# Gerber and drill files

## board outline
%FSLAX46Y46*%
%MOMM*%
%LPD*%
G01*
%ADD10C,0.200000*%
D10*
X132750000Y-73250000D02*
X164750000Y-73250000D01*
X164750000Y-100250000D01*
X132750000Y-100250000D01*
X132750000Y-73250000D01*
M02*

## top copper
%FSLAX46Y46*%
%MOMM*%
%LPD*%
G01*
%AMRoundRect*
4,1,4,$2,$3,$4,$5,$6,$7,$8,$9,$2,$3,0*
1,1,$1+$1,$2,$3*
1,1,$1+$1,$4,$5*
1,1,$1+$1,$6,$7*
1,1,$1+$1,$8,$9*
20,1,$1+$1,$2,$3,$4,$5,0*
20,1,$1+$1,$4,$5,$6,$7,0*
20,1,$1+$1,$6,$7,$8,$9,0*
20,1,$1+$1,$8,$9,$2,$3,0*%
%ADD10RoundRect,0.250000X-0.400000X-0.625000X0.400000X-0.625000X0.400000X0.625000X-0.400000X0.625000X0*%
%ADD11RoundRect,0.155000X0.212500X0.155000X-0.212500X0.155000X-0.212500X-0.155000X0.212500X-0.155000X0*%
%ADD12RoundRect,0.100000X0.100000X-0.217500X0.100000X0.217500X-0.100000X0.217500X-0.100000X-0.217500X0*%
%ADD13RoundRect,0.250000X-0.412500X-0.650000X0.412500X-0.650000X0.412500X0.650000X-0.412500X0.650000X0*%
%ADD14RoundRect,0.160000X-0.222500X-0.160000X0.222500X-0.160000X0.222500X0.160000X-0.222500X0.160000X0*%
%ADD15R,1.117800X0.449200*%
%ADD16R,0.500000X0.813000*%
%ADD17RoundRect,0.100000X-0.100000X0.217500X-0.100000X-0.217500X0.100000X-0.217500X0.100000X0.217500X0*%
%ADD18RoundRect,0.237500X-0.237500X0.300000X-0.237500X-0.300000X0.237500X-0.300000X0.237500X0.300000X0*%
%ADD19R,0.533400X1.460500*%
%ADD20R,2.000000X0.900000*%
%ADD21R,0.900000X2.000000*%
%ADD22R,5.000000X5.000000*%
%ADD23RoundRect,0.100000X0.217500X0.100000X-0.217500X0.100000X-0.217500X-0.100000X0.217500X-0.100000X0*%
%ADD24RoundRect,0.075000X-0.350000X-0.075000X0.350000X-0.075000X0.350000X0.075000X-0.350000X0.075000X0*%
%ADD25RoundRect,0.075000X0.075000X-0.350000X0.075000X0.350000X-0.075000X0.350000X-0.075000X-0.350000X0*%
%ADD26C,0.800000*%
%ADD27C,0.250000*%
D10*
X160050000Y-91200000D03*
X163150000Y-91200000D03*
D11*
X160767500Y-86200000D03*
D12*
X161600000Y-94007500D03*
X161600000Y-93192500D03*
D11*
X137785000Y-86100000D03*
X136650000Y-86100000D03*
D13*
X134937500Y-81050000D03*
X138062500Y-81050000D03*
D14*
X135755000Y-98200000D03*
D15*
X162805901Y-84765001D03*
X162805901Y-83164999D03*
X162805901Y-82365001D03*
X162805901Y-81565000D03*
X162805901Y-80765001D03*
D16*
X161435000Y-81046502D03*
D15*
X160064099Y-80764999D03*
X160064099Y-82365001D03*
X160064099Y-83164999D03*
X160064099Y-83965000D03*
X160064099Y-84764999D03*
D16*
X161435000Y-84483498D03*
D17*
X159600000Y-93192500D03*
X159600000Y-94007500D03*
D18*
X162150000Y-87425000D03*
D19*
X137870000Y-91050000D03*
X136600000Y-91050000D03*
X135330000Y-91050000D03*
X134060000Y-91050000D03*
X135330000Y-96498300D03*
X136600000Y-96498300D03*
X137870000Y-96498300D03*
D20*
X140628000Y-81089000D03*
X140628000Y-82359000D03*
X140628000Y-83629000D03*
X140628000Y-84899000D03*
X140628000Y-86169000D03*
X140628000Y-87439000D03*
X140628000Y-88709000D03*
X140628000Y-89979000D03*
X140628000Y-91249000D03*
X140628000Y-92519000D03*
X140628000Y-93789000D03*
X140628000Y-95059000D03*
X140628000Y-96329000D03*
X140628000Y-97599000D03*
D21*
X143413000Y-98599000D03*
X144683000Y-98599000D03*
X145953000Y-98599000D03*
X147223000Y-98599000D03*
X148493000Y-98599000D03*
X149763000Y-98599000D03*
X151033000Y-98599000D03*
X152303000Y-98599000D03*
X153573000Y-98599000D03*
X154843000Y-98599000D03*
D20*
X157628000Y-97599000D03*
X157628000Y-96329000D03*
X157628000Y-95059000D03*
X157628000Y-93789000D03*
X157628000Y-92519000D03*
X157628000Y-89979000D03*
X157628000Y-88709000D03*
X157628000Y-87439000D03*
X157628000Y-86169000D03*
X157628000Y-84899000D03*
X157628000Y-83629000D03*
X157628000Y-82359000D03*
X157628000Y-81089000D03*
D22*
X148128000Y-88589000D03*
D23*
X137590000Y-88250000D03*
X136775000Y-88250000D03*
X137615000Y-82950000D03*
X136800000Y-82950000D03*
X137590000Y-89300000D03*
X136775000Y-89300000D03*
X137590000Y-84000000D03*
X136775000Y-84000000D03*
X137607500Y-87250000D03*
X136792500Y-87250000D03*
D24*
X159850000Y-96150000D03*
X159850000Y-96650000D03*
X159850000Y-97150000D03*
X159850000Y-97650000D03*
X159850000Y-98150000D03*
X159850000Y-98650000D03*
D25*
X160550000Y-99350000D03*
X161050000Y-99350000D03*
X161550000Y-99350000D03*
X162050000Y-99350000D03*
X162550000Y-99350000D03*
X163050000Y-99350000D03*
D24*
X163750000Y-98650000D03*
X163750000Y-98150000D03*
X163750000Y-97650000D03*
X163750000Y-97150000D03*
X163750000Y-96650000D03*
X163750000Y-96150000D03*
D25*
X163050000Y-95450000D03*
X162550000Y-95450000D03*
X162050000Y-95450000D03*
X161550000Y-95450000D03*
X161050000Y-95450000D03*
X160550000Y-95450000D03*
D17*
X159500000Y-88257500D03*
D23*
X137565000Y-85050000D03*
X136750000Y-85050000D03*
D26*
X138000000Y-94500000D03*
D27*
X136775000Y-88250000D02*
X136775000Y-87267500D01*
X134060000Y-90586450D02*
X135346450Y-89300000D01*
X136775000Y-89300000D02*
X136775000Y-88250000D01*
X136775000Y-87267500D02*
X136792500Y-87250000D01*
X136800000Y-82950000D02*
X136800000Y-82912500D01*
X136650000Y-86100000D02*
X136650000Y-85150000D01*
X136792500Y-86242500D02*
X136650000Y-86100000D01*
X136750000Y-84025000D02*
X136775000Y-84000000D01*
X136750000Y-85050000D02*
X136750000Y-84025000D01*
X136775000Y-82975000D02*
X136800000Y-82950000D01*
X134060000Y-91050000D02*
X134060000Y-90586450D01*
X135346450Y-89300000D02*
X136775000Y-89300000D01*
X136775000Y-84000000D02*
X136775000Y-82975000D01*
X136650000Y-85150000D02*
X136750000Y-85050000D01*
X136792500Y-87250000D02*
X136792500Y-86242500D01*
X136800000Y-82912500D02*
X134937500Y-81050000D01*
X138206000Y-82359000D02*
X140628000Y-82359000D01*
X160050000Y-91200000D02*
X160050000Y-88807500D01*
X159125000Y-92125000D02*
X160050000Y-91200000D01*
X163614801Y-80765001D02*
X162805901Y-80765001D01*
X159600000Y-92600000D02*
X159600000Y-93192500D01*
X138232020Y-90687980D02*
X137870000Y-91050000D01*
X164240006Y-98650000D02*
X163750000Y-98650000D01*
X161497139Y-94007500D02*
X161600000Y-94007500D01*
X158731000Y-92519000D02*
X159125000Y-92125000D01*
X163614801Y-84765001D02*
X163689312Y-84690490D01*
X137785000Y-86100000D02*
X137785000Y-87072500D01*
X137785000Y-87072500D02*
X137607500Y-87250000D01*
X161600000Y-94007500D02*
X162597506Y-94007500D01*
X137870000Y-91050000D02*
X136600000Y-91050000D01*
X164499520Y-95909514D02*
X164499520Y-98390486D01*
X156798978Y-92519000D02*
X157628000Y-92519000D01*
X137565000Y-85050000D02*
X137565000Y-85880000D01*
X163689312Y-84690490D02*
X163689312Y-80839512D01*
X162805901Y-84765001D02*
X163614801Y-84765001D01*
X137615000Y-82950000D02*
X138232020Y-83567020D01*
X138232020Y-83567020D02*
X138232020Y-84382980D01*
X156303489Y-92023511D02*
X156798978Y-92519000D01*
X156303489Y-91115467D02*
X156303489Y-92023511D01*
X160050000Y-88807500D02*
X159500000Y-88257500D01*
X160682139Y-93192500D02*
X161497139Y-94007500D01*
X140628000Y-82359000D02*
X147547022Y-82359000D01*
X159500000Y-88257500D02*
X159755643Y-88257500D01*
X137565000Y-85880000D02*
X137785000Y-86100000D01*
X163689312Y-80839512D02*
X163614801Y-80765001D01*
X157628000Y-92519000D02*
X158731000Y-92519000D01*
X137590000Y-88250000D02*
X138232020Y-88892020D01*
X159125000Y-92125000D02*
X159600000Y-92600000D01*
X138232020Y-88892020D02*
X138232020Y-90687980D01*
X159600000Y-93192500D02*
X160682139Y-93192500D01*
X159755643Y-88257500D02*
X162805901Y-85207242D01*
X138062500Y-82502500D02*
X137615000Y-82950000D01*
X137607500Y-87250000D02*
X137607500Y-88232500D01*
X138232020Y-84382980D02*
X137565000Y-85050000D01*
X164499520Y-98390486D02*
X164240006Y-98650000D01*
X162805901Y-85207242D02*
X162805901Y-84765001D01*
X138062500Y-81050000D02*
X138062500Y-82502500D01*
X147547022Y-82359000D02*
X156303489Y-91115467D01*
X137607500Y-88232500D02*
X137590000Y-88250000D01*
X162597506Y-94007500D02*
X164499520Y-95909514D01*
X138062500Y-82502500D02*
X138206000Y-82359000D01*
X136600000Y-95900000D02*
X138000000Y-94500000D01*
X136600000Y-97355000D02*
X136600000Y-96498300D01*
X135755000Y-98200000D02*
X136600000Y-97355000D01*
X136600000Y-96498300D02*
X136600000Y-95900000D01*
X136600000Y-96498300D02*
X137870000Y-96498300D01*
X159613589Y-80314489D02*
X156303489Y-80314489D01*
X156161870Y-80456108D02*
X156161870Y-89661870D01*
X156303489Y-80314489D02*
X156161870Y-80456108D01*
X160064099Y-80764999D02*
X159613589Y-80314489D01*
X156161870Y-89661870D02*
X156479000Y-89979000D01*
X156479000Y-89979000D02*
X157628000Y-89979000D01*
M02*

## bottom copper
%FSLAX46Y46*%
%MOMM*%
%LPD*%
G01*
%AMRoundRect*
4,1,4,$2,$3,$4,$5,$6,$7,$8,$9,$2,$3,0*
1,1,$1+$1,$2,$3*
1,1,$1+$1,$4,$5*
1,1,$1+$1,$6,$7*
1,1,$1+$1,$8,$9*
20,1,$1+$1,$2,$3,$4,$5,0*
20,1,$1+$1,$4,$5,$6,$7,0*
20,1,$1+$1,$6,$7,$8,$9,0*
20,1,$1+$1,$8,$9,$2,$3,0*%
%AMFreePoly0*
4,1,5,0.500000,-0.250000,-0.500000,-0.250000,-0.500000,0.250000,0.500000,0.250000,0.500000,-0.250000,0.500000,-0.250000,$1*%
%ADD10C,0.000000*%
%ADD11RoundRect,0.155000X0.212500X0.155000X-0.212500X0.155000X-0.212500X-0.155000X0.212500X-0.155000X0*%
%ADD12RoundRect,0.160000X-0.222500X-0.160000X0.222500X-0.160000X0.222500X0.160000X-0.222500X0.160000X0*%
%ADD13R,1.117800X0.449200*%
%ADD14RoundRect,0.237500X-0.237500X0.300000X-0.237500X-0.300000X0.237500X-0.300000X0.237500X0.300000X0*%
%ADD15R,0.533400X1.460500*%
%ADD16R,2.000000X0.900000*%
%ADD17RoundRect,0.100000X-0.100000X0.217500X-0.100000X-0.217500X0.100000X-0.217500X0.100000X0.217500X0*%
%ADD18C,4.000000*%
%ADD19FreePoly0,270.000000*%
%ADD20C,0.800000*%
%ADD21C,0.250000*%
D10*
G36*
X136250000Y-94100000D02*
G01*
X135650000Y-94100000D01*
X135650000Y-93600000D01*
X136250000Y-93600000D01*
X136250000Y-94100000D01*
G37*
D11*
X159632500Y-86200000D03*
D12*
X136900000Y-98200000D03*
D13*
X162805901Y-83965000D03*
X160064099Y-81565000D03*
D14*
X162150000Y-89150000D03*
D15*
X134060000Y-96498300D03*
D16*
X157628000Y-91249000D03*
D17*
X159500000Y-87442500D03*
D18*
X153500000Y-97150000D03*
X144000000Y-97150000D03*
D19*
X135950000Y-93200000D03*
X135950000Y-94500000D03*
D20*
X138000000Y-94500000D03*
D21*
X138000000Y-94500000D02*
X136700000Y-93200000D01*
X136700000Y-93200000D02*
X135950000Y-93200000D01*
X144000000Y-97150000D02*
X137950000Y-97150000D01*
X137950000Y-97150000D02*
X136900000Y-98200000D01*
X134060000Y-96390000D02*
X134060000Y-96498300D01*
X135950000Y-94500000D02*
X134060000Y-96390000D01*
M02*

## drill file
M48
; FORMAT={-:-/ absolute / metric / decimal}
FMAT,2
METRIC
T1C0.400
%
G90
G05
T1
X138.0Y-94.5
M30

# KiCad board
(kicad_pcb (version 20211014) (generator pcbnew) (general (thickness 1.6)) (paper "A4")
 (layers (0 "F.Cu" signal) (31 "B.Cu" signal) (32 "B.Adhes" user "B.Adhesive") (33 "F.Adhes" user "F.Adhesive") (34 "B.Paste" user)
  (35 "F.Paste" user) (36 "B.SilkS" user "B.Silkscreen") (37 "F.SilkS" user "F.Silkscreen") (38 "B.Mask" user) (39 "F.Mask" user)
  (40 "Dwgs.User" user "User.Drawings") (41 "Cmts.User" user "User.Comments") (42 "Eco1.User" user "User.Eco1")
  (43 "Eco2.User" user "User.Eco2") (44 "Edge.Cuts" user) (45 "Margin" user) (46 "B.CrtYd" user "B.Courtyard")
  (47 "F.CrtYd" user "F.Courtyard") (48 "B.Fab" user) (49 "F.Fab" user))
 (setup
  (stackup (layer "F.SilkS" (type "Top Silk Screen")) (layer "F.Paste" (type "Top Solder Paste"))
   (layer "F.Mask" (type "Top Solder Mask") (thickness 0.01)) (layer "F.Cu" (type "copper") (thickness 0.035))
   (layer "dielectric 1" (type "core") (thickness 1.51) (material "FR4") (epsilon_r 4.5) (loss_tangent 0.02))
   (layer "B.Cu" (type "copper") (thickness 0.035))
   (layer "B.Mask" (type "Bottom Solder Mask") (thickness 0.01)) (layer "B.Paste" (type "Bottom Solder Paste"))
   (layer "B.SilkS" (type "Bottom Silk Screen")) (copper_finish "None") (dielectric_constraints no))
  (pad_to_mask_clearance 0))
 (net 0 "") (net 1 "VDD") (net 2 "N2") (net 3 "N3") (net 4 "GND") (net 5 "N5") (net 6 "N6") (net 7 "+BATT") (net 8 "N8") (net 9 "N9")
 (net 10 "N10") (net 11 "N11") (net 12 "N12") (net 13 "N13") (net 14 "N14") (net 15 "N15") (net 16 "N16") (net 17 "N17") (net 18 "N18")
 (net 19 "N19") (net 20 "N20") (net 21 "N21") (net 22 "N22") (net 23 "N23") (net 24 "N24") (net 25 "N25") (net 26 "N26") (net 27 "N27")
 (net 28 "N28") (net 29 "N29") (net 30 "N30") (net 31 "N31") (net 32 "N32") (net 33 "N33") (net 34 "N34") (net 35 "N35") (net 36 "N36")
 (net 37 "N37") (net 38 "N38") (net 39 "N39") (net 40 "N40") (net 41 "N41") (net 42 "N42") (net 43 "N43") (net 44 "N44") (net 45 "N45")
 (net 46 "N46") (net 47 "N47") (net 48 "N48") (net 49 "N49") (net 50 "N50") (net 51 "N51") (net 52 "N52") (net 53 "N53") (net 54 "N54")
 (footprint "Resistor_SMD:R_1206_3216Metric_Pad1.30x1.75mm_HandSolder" (layer "F.Cu") (at 161.6 91.2)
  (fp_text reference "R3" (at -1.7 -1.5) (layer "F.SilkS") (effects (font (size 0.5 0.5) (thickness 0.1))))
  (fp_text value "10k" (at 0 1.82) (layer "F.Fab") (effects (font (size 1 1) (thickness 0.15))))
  (pad "1" smd roundrect (at -1.55 0) (size 1.3 1.75) (layers "F.Cu" "F.Paste" "F.Mask") (roundrect_rratio 0.192308) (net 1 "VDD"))
  (pad "2" smd roundrect (at 1.55 0) (size 1.3 1.75) (layers "F.Cu" "F.Paste" "F.Mask") (roundrect_rratio 0.192308) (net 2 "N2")))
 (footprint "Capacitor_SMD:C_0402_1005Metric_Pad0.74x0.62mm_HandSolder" (layer "F.Cu") (at 160.2 86.2 180)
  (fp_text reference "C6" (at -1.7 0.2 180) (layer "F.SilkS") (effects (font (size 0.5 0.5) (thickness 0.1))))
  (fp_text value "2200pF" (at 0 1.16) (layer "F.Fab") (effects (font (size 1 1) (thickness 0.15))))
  (pad "1" smd roundrect (at -0.5675 0 180) (size 0.735 0.62) (layers "F.Cu" "F.Paste" "F.Mask") (roundrect_rratio 0.25) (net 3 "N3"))
  (pad "2" smd roundrect (at 0.5675 0 180) (size 0.735 0.62) (layers "B.Cu" "F.Paste" "F.Mask") (roundrect_rratio 0.25) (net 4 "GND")))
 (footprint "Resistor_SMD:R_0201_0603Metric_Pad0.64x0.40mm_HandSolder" (layer "F.Cu") (at 161.6 93.6 90)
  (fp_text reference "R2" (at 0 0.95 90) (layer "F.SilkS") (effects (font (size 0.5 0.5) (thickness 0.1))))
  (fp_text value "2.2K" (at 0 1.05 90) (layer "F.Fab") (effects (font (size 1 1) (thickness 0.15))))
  (pad "" smd roundrect (at -0.4325 0 90) (size 0.458 0.36) (layers "F.Paste") (roundrect_rratio 0.25))
  (pad "" smd roundrect (at 0.4325 0 90) (size 0.458 0.36) (layers "F.Paste") (roundrect_rratio 0.25))
  (pad "1" smd roundrect (at -0.4075 0 90) (size 0.635 0.4) (layers "F.Cu" "F.Mask") (roundrect_rratio 0.25) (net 1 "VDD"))
  (pad "2" smd roundrect (at 0.4075 0 90) (size 0.635 0.4) (layers "F.Cu" "F.Mask") (roundrect_rratio 0.25) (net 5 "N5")))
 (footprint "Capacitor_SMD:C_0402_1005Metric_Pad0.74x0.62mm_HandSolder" (layer "F.Cu") (at 137.2175 86.1 180)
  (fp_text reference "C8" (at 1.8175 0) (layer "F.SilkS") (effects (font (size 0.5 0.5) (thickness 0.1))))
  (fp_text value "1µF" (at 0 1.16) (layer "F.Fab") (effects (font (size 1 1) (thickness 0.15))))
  (pad "1" smd roundrect (at -0.5675 0 180) (size 0.735 0.62) (layers "F.Cu" "F.Paste" "F.Mask") (roundrect_rratio 0.25) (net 1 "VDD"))
  (pad "2" smd roundrect (at 0.5675 0 180) (size 0.735 0.62) (layers "F.Cu" "F.Paste" "F.Mask") (roundrect_rratio 0.25) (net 4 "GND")))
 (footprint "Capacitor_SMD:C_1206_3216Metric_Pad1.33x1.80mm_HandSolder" (layer "F.Cu") (at 136.5 81.05)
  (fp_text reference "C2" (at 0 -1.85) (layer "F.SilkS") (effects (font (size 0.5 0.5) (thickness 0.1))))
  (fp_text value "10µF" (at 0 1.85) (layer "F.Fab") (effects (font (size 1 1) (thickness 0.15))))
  (pad "1" smd roundrect (at -1.5625 0) (size 1.325 1.8) (layers "F.Cu" "F.Paste" "F.Mask") (roundrect_rratio 0.188679) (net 4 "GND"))
  (pad "2" smd roundrect (at 1.5625 0) (size 1.325 1.8) (layers "F.Cu" "F.Paste" "F.Mask") (roundrect_rratio 0.188679) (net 1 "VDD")))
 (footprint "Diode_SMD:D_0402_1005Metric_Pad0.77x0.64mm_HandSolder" (layer "F.Cu") (at 136.3275 98.2)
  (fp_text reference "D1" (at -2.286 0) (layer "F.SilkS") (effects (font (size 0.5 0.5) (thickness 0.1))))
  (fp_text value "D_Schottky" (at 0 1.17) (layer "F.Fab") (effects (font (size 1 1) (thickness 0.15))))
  (pad "1" smd roundrect (at -0.5725 0) (size 0.765 0.64) (layers "F.Cu" "F.Paste" "F.Mask") (roundrect_rratio 0.25) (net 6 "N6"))
  (pad "2" smd roundrect (at 0.5725 0) (size 0.765 0.64) (layers "B.Cu" "F.Paste" "F.Mask") (roundrect_rratio 0.25) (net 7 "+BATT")))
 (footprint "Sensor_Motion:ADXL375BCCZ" (layer "F.Cu") (at 161.435 82.765 180)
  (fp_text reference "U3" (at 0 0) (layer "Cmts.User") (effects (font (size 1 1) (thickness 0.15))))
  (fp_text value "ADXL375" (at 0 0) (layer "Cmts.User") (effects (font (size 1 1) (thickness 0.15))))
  (pad "1" smd rect (at -1.370901 -2.000001 270) (size 0.4492 1.1178) (layers "F.Cu" "F.Paste" "F.Mask") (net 1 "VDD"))
  (pad "2" smd rect (at -1.370901 -1.2 270) (size 0.4492 1.1178) (layers "B.Cu" "F.Paste" "F.Mask") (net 4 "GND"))
  (pad "3" smd rect (at -1.370901 -0.399999 270) (size 0.4492 1.1178) (layers "F.Cu" "F.Paste" "F.Mask") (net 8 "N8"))
  (pad "4" smd rect (at -1.370901 0.399999 270) (size 0.4492 1.1178) (layers "F.Cu" "F.Paste" "F.Mask") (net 4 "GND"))
  (pad "5" smd rect (at -1.370901 1.2 270) (size 0.4492 1.1178) (layers "F.Cu" "F.Paste" "F.Mask") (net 4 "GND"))
  (pad "6" smd rect (at -1.370901 1.999999 270) (size 0.4492 1.1178) (layers "F.Cu" "F.Paste" "F.Mask") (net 1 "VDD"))
  (pad "7" smd rect (at 0 1.718498 180) (size 0.5 0.813) (layers "F.Cu" "F.Paste" "F.Mask") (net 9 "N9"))
  (pad "8" smd rect (at 1.370901 2.000001 270) (size 0.4492 1.1178) (layers "F.Cu" "F.Paste" "F.Mask") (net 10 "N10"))
  (pad "9" smd rect (at 1.370901 1.2 270) (size 0.4492 1.1178) (layers "B.Cu" "F.Paste" "F.Mask") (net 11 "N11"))
  (pad "10" smd rect (at 1.370901 0.399999 270) (size 0.4492 1.1178) (layers "F.Cu" "F.Paste" "F.Mask") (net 4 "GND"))
  (pad "11" smd rect (at 1.370901 -0.399999 270) (size 0.4492 1.1178) (layers "F.Cu" "F.Paste" "F.Mask") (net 4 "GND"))
  (pad "12" smd rect (at 1.370901 -1.2 270) (size 0.4492 1.1178) (layers "F.Cu" "F.Paste" "F.Mask") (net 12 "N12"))
  (pad "13" smd rect (at 1.370901 -1.999999 270) (size 0.4492 1.1178) (layers "F.Cu" "F.Paste" "F.Mask") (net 5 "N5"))
  (pad "14" smd rect (at 0 -1.718498 180) (size 0.5 0.813) (layers "F.Cu" "F.Paste" "F.Mask") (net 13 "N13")))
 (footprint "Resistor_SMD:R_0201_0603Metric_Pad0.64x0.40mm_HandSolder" (layer "F.Cu") (at 159.6 93.6 -90)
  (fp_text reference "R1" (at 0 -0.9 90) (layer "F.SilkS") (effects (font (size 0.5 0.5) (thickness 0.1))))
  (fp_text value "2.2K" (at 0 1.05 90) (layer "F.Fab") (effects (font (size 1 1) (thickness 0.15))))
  (pad "" smd roundrect (at 0.4325 0 270) (size 0.458 0.36) (layers "F.Paste") (roundrect_rratio 0.25))
  (pad "" smd roundrect (at -0.4325 0 270) (size 0.458 0.36) (layers "F.Paste") (roundrect_rratio 0.25))
  (pad "1" smd roundrect (at -0.4075 0 270) (size 0.635 0.4) (layers "F.Cu" "F.Mask") (roundrect_rratio 0.25) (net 1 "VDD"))
  (pad "2" smd roundrect (at 0.4075 0 270) (size 0.635 0.4) (layers "F.Cu" "F.Mask") (roundrect_rratio 0.25) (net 13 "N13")))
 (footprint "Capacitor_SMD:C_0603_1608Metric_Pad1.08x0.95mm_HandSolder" (layer "F.Cu") (at 162.15 88.2875 -90)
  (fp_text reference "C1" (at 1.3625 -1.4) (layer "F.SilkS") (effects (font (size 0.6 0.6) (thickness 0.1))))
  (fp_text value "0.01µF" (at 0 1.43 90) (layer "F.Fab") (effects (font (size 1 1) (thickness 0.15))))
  (pad "1" smd roundrect (at -0.8625 0 270) (size 1.075 0.95) (layers "F.Cu" "F.Paste" "F.Mask") (roundrect_rratio 0.25) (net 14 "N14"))
  (pad "2" smd roundrect (at 0.8625 0 270) (size 1.075 0.95) (layers "B.Cu" "F.Paste" "F.Mask") (roundrect_rratio 0.25) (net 4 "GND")))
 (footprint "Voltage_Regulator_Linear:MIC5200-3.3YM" (layer "F.Cu") (at 135.965 93.77415 -90)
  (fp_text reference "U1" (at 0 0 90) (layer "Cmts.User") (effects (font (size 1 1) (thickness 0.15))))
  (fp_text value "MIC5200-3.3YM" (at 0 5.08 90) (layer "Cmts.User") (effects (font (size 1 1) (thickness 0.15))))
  (pad "1" smd rect (at -2.72415 -1.905 270) (size 1.4605 0.5334) (layers "F.Cu" "F.Paste" "F.Mask") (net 1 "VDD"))
  (pad "2" smd rect (at -2.72415 -0.635 270) (size 1.4605 0.5334) (layers "F.Cu" "F.Paste" "F.Mask") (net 1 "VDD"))
  (pad "3" smd rect (at -2.72415 0.635 270) (size 1.4605 0.5334) (layers "F.Cu" "F.Paste" "F.Mask") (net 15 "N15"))
  (pad "4" smd rect (at -2.72415 1.905 270) (size 1.4605 0.5334) (layers "F.Cu" "F.Paste" "F.Mask") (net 4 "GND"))
  (pad "5" smd rect (at 2.72415 1.905 270) (size 1.4605 0.5334) (layers "B.Cu" "F.Paste" "F.Mask") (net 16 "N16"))
  (pad "6" smd rect (at 2.72415 0.635 270) (size 1.4605 0.5334) (layers "F.Cu" "F.Paste" "F.Mask") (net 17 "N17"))
  (pad "7" smd rect (at 2.72415 -0.635 270) (size 1.4605 0.5334) (layers "F.Cu" "F.Paste" "F.Mask") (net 6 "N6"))
  (pad "8" smd rect (at 2.72415 -1.905 270) (size 1.4605 0.5334) (layers "F.Cu" "F.Paste" "F.Mask") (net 6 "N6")))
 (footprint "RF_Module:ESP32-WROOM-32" (layer "F.Cu") (at 149.128 89.344)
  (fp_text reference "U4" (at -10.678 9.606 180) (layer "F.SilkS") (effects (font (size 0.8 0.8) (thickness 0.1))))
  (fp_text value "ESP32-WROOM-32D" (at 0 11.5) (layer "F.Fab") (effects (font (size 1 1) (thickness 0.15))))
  (pad "1" smd rect (at -8.5 -8.255) (size 2 0.9) (layers "F.Cu" "F.Paste" "F.Mask") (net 4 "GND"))
  (pad "2" smd rect (at -8.5 -6.985) (size 2 0.9) (layers "F.Cu" "F.Paste" "F.Mask") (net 1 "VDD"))
  (pad "3" smd rect (at -8.5 -5.715) (size 2 0.9) (layers "F.Cu" "F.Paste" "F.Mask") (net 2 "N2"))
  (pad "4" smd rect (at -8.5 -4.445) (size 2 0.9) (layers "F.Cu" "F.Paste" "F.Mask") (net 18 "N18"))
  (pad "5" smd rect (at -8.5 -3.175) (size 2 0.9) (layers "F.Cu" "F.Paste" "F.Mask") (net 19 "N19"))
  (pad "6" smd rect (at -8.5 -1.905) (size 2 0.9) (layers "F.Cu" "F.Paste" "F.Mask") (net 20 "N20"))
  (pad "7" smd rect (at -8.5 -0.635) (size 2 0.9) (layers "F.Cu" "F.Paste" "F.Mask") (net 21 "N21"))
  (pad "8" smd rect (at -8.5 0.635) (size 2 0.9) (layers "F.Cu" "F.Paste" "F.Mask") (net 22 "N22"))
  (pad "9" smd rect (at -8.5 1.905) (size 2 0.9) (layers "F.Cu" "F.Paste" "F.Mask") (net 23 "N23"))
  (pad "10" smd rect (at -8.5 3.175) (size 2 0.9) (layers "F.Cu" "F.Paste" "F.Mask") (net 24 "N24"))
  (pad "11" smd rect (at -8.5 4.445) (size 2 0.9) (layers "F.Cu" "F.Paste" "F.Mask") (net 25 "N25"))
  (pad "12" smd rect (at -8.5 5.715) (size 2 0.9) (layers "F.Cu" "F.Paste" "F.Mask") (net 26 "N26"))
  (pad "13" smd rect (at -8.5 6.985) (size 2 0.9) (layers "F.Cu" "F.Paste" "F.Mask") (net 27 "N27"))
  (pad "14" smd rect (at -8.5 8.255) (size 2 0.9) (layers "F.Cu" "F.Paste" "F.Mask") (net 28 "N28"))
  (pad "15" smd rect (at -5.715 9.255 90) (size 2 0.9) (layers "F.Cu" "F.Paste" "F.Mask") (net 4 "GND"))
  (pad "16" smd rect (at -4.445 9.255 90) (size 2 0.9) (layers "F.Cu" "F.Paste" "F.Mask") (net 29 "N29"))
  (pad "17" smd rect (at -3.175 9.255 90) (size 2 0.9) (layers "F.Cu" "F.Paste" "F.Mask") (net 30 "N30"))
  (pad "18" smd rect (at -1.905 9.255 90) (size 2 0.9) (layers "F.Cu" "F.Paste" "F.Mask") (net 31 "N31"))
  (pad "19" smd rect (at -0.635 9.255 90) (size 2 0.9) (layers "F.Cu" "F.Paste" "F.Mask") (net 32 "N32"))
  (pad "20" smd rect (at 0.635 9.255 90) (size 2 0.9) (layers "F.Cu" "F.Paste" "F.Mask") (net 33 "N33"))
  (pad "21" smd rect (at 1.905 9.255 90) (size 2 0.9) (layers "F.Cu" "F.Paste" "F.Mask") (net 5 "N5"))
  (pad "22" smd rect (at 3.175 9.255 90) (size 2 0.9) (layers "F.Cu" "F.Paste" "F.Mask") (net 13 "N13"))
  (pad "23" smd rect (at 4.445 9.255 90) (size 2 0.9) (layers "F.Cu" "F.Paste" "F.Mask") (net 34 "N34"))
  (pad "24" smd rect (at 5.715 9.255 90) (size 2 0.9) (layers "F.Cu" "F.Paste" "F.Mask") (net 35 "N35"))
  (pad "25" smd rect (at 8.5 8.255) (size 2 0.9) (layers "F.Cu" "F.Paste" "F.Mask") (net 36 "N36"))
  (pad "26" smd rect (at 8.5 6.985) (size 2 0.9) (layers "F.Cu" "F.Paste" "F.Mask") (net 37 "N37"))
  (pad "27" smd rect (at 8.5 5.715) (size 2 0.9) (layers "F.Cu" "F.Paste" "F.Mask") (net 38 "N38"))
  (pad "28" smd rect (at 8.5 4.445) (size 2 0.9) (layers "F.Cu" "F.Paste" "F.Mask") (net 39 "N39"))
  (pad "29" smd rect (at 8.5 3.175) (size 2 0.9) (layers "F.Cu" "F.Paste" "F.Mask") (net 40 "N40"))
  (pad "30" smd rect (at 8.5 1.905) (size 2 0.9) (layers "B.Cu" "F.Paste" "F.Mask") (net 11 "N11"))
  (pad "31" smd rect (at 8.5 0.635) (size 2 0.9) (layers "F.Cu" "F.Paste" "F.Mask") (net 10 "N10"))
  (pad "32" smd rect (at 8.5 -0.635) (size 2 0.9) (layers "F.Cu" "F.Paste" "F.Mask") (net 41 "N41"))
  (pad "33" smd rect (at 8.5 -1.905) (size 2 0.9) (layers "F.Cu" "F.Paste" "F.Mask") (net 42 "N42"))
  (pad "34" smd rect (at 8.5 -3.175) (size 2 0.9) (layers "F.Cu" "F.Paste" "F.Mask") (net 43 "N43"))
  (pad "35" smd rect (at 8.5 -4.445) (size 2 0.9) (layers "F.Cu" "F.Paste" "F.Mask") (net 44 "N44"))
  (pad "36" smd rect (at 8.5 -5.715) (size 2 0.9) (layers "F.Cu" "F.Paste" "F.Mask") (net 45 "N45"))
  (pad "37" smd rect (at 8.5 -6.985) (size 2 0.9) (layers "F.Cu" "F.Paste" "F.Mask") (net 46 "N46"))
  (pad "38" smd rect (at 8.5 -8.255) (size 2 0.9) (layers "F.Cu" "F.Paste" "F.Mask") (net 4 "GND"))
  (pad "39" smd rect (at -1 -0.755) (size 5 5) (layers "F.Cu" "F.Paste" "F.Mask") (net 4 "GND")))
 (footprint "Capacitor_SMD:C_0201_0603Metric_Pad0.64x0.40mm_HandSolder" (layer "F.Cu") (at 137.1825 88.25 180)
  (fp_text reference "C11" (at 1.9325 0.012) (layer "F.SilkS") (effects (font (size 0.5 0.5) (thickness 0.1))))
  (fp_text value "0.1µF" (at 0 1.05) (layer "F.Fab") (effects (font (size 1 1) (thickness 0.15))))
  (pad "" smd roundrect (at -0.4325 0 180) (size 0.458 0.36) (layers "F.Paste") (roundrect_rratio 0.25))
  (pad "" smd roundrect (at 0.4325 0 180) (size 0.458 0.36) (layers "F.Paste") (roundrect_rratio 0.25))
  (pad "1" smd roundrect (at -0.4075 0 180) (size 0.635 0.4) (layers "F.Cu" "F.Mask") (roundrect_rratio 0.25) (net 1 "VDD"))
  (pad "2" smd roundrect (at 0.4075 0 180) (size 0.635 0.4) (layers "F.Cu" "F.Mask") (roundrect_rratio 0.25) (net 4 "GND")))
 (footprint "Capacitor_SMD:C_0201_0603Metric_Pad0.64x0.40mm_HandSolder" (layer "F.Cu") (at 137.2075 82.95 180)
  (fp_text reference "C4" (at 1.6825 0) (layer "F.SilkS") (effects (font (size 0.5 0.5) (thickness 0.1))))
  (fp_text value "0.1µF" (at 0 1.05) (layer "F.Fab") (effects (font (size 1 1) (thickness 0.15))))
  (pad "" smd roundrect (at 0.4325 0 180) (size 0.458 0.36) (layers "F.Paste") (roundrect_rratio 0.25))
  (pad "" smd roundrect (at -0.4325 0 180) (size 0.458 0.36) (layers "F.Paste") (roundrect_rratio 0.25))
  (pad "1" smd roundrect (at -0.4075 0 180) (size 0.635 0.4) (layers "F.Cu" "F.Mask") (roundrect_rratio 0.25) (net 1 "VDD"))
  (pad "2" smd roundrect (at 0.4075 0 180) (size 0.635 0.4) (layers "F.Cu" "F.Mask") (roundrect_rratio 0.25) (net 4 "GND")))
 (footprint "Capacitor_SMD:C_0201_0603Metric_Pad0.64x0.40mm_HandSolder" (layer "F.Cu") (at 137.1825 89.3 180)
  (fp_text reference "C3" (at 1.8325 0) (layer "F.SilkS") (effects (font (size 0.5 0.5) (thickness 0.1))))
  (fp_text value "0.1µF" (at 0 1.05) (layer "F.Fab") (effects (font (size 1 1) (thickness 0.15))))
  (pad "" smd roundrect (at -0.4325 0 180) (size 0.458 0.36) (layers "F.Paste") (roundrect_rratio 0.25))
  (pad "" smd roundrect (at 0.4325 0 180) (size 0.458 0.36) (layers "F.Paste") (roundrect_rratio 0.25))
  (pad "1" smd roundrect (at -0.4075 0 180) (size 0.635 0.4) (layers "F.Cu" "F.Mask") (roundrect_rratio 0.25) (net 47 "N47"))
  (pad "2" smd roundrect (at 0.4075 0 180) (size 0.635 0.4) (layers "F.Cu" "F.Mask") (roundrect_rratio 0.25) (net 4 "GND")))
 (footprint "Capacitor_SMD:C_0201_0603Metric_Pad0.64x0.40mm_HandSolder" (layer "F.Cu") (at 137.1825 84 180)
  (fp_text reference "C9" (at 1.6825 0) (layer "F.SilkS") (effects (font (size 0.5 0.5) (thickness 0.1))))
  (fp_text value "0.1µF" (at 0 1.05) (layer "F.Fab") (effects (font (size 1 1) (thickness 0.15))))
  (pad "" smd roundrect (at -0.4325 0 180) (size 0.458 0.36) (layers "F.Paste") (roundrect_rratio 0.25))
  (pad "" smd roundrect (at 0.4325 0 180) (size 0.458 0.36) (layers "F.Paste") (roundrect_rratio 0.25))
  (pad "1" smd roundrect (at -0.4075 0 180) (size 0.635 0.4) (layers "F.Cu" "F.Mask") (roundrect_rratio 0.25) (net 2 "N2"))
  (pad "2" smd roundrect (at 0.4075 0 180) (size 0.635 0.4) (layers "F.Cu" "F.Mask") (roundrect_rratio 0.25) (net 4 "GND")))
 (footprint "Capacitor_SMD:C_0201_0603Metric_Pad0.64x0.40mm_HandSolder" (layer "F.Cu") (at 137.2 87.25 180)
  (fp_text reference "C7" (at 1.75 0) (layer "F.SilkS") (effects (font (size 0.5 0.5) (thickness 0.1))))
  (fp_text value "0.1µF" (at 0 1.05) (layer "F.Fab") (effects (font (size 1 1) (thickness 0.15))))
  (pad "" smd roundrect (at 0.4325 0 180) (size 0.458 0.36) (layers "F.Paste") (roundrect_rratio 0.25))
  (pad "" smd roundrect (at -0.4325 0 180) (size 0.458 0.36) (layers "F.Paste") (roundrect_rratio 0.25))
  (pad "1" smd roundrect (at -0.4075 0 180) (size 0.635 0.4) (layers "F.Cu" "F.Mask") (roundrect_rratio 0.25) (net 1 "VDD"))
  (pad "2" smd roundrect (at 0.4075 0 180) (size 0.635 0.4) (layers "F.Cu" "F.Mask") (roundrect_rratio 0.25) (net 4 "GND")))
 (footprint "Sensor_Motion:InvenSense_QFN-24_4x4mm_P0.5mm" (layer "F.Cu") (at 161.8 97.4)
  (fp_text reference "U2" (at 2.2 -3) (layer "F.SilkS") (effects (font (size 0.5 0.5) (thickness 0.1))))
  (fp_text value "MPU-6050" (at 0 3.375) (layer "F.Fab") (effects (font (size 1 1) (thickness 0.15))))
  (pad "1" smd roundrect (at -1.95 -1.25) (size 0.85 0.3) (layers "F.Cu" "F.Paste" "F.Mask") (roundrect_rratio 0.25) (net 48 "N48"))
  (pad "2" smd roundrect (at -1.95 -0.75) (size 0.85 0.3) (layers "F.Cu" "F.Paste" "F.Mask") (roundrect_rratio 0.25))
  (pad "3" smd roundrect (at -1.95 -0.25) (size 0.85 0.3) (layers "F.Cu" "F.Paste" "F.Mask") (roundrect_rratio 0.25))
  (pad "4" smd roundrect (at -1.95 0.25) (size 0.85 0.3) (layers "F.Cu" "F.Paste" "F.Mask") (roundrect_rratio 0.25))
  (pad "5" smd roundrect (at -1.95 0.75) (size 0.85 0.3) (layers "F.Cu" "F.Paste" "F.Mask") (roundrect_rratio 0.25))
  (pad "6" smd roundrect (at -1.95 1.25) (size 0.85 0.3) (layers "F.Cu" "F.Paste" "F.Mask") (roundrect_rratio 0.25) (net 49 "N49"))
  (pad "7" smd roundrect (at -1.25 1.95 90) (size 0.85 0.3) (layers "F.Cu" "F.Paste" "F.Mask") (roundrect_rratio 0.25) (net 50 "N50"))
  (pad "8" smd roundrect (at -0.75 1.95 90) (size 0.85 0.3) (layers "F.Cu" "F.Paste" "F.Mask") (roundrect_rratio 0.25) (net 14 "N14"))
  (pad "9" smd roundrect (at -0.25 1.95 90) (size 0.85 0.3) (layers "F.Cu" "F.Paste" "F.Mask") (roundrect_rratio 0.25) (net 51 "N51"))
  (pad "10" smd roundrect (at 0.25 1.95 90) (size 0.85 0.3) (layers "F.Cu" "F.Paste" "F.Mask") (roundrect_rratio 0.25) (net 47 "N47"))
  (pad "11" smd roundrect (at 0.75 1.95 90) (size 0.85 0.3) (layers "F.Cu" "F.Paste" "F.Mask") (roundrect_rratio 0.25) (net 4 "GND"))
  (pad "12" smd roundrect (at 1.25 1.95 90) (size 0.85 0.3) (layers "F.Cu" "F.Paste" "F.Mask") (roundrect_rratio 0.25) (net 40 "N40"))
  (pad "13" smd roundrect (at 1.95 1.25) (size 0.85 0.3) (layers "F.Cu" "F.Paste" "F.Mask") (roundrect_rratio 0.25) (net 1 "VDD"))
  (pad "14" smd roundrect (at 1.95 0.75) (size 0.85 0.3) (layers "F.Cu" "F.Paste" "F.Mask") (roundrect_rratio 0.25))
  (pad "15" smd roundrect (at 1.95 0.25) (size 0.85 0.3) (layers "F.Cu" "F.Paste" "F.Mask") (roundrect_rratio 0.25))
  (pad "16" smd roundrect (at 1.95 -0.25) (size 0.85 0.3) (layers "F.Cu" "F.Paste" "F.Mask") (roundrect_rratio 0.25))
  (pad "17" smd roundrect (at 1.95 -0.75) (size 0.85 0.3) (layers "F.Cu" "F.Paste" "F.Mask") (roundrect_rratio 0.25))
  (pad "18" smd roundrect (at 1.95 -1.25) (size 0.85 0.3) (layers "F.Cu" "F.Paste" "F.Mask") (roundrect_rratio 0.25) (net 4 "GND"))
  (pad "19" smd roundrect (at 1.25 -1.95 90) (size 0.85 0.3) (layers "F.Cu" "F.Paste" "F.Mask") (roundrect_rratio 0.25) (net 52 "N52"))
  (pad "20" smd roundrect (at 0.75 -1.95 90) (size 0.85 0.3) (layers "F.Cu" "F.Paste" "F.Mask") (roundrect_rratio 0.25) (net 3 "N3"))
  (pad "21" smd roundrect (at 0.25 -1.95 90) (size 0.85 0.3) (layers "F.Cu" "F.Paste" "F.Mask") (roundrect_rratio 0.25) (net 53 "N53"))
  (pad "22" smd roundrect (at -0.25 -1.95 90) (size 0.85 0.3) (layers "F.Cu" "F.Paste" "F.Mask") (roundrect_rratio 0.25) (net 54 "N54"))
  (pad "23" smd roundrect (at -0.75 -1.95 90) (size 0.85 0.3) (layers "F.Cu" "F.Paste" "F.Mask") (roundrect_rratio 0.25) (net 13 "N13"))
  (pad "24" smd roundrect (at -1.25 -1.95 90) (size 0.85 0.3) (layers "F.Cu" "F.Paste" "F.Mask") (roundrect_rratio 0.25) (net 5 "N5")))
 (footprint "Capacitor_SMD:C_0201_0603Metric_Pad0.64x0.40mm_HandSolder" (layer "F.Cu") (at 159.5 87.85 -90)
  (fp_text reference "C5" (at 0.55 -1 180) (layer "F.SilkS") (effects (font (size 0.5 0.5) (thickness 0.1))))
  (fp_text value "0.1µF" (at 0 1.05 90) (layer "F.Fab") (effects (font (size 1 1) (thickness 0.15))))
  (pad "" smd roundrect (at 0.4325 0 270) (size 0.458 0.36) (layers "F.Paste") (roundrect_rratio 0.25))
  (pad "" smd roundrect (at -0.4325 0 270) (size 0.458 0.36) (layers "F.Paste") (roundrect_rratio 0.25))
  (pad "1" smd roundrect (at -0.4075 0 270) (size 0.635 0.4) (layers "B.Cu" "F.Mask") (roundrect_rratio 0.25) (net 4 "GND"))
  (pad "2" smd roundrect (at 0.4075 0 270) (size 0.635 0.4) (layers "F.Cu" "F.Mask") (roundrect_rratio 0.25) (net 1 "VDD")))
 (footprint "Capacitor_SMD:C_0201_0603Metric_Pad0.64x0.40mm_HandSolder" (layer "F.Cu") (at 137.1575 85.05 180)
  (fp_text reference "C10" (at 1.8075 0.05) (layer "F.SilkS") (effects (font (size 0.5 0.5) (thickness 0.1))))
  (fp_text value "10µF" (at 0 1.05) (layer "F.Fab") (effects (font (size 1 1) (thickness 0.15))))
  (pad "" smd roundrect (at 0.4325 0 180) (size 0.458 0.36) (layers "F.Paste") (roundrect_rratio 0.25))
  (pad "" smd roundrect (at -0.4325 0 180) (size 0.458 0.36) (layers "F.Paste") (roundrect_rratio 0.25))
  (pad "1" smd roundrect (at -0.4075 0 180) (size 0.635 0.4) (layers "F.Cu" "F.Mask") (roundrect_rratio 0.25) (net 1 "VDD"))
  (pad "2" smd roundrect (at 0.4075 0 180) (size 0.635 0.4) (layers "F.Cu" "F.Mask") (roundrect_rratio 0.25) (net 4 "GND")))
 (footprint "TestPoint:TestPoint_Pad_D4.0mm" (layer "B.Cu") (at 153.5 97.15 180)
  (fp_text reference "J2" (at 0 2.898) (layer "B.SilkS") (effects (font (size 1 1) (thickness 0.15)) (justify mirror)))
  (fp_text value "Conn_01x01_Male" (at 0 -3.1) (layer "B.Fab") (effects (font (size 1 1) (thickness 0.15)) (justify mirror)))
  (pad "1" smd circle (at 0 0 180) (size 4 4) (layers "B.Cu" "B.Mask") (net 4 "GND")))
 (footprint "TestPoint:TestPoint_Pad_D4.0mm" (layer "B.Cu") (at 144 97.15 180)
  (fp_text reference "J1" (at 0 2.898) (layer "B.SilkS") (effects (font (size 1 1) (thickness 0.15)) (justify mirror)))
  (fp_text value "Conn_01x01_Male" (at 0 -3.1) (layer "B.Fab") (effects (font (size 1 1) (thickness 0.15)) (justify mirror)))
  (pad "1" smd circle (at 0 0 180) (size 4 4) (layers "B.Cu" "B.Mask") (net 7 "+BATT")))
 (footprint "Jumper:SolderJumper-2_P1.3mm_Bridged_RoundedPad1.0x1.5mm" (layer "B.Cu") (at 135.95 93.85 -90)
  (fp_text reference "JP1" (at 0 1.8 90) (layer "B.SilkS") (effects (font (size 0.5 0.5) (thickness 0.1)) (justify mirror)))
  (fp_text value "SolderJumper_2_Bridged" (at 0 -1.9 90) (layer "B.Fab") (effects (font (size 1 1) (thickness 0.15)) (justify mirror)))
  (fp_poly (pts (xy 0.25 0.3) (xy -0.25 0.3) (xy -0.25 -0.3) (xy 0.25 -0.3)) (layer "B.Cu") (width 0) (fill solid))
  (pad "1" smd custom (at -0.65 0 270) (size 1 0.5) (layers "B.Cu" "B.Mask") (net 6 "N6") (zone_connect 2)
   (options (clearance outline) (anchor rect)) (primitives))
  (pad "2" smd custom (at 0.65 0 270) (size 1 0.5) (layers "B.Cu" "B.Mask") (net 16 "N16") (zone_connect 2)
   (options (clearance outline) (anchor rect)) (primitives)))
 (gr_rect (start 132.75 100.25) (end 164.75 73.25) (layer "Edge.Cuts") (width 0.2) (fill none))
 (segment (start 136.775 88.25) (end 136.775 87.2675) (width 0.25) (layer "F.Cu") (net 4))
 (segment (start 134.06 90.58645) (end 135.34645 89.3) (width 0.25) (layer "F.Cu") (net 4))
 (segment (start 136.775 89.3) (end 136.775 88.25) (width 0.25) (layer "F.Cu") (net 4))
 (segment (start 136.775 87.2675) (end 136.7925 87.25) (width 0.25) (layer "F.Cu") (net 4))
 (segment (start 136.8 82.95) (end 136.8 82.9125) (width 0.25) (layer "F.Cu") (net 4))
 (segment (start 136.65 86.1) (end 136.65 85.15) (width 0.25) (layer "F.Cu") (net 4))
 (segment (start 136.7925 86.2425) (end 136.65 86.1) (width 0.25) (layer "F.Cu") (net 4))
 (segment (start 136.75 84.025) (end 136.775 84) (width 0.25) (layer "F.Cu") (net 4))
 (segment (start 136.75 85.05) (end 136.75 84.025) (width 0.25) (layer "F.Cu") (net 4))
 (segment (start 136.775 82.975) (end 136.8 82.95) (width 0.25) (layer "F.Cu") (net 4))
 (segment (start 134.06 91.05) (end 134.06 90.58645) (width 0.25) (layer "F.Cu") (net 4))
 (segment (start 135.34645 89.3) (end 136.775 89.3) (width 0.25) (layer "F.Cu") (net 4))
 (segment (start 136.775 84) (end 136.775 82.975) (width 0.25) (layer "F.Cu") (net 4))
 (segment (start 136.65 85.15) (end 136.75 85.05) (width 0.25) (layer "F.Cu") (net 4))
 (segment (start 136.7925 87.25) (end 136.7925 86.2425) (width 0.25) (layer "F.Cu") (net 4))
 (segment (start 136.8 82.9125) (end 134.9375 81.05) (width 0.25) (layer "F.Cu") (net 4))
 (segment (start 138.206 82.359) (end 140.628 82.359) (width 0.25) (layer "F.Cu") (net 1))
 (segment (start 160.05 91.2) (end 160.05 88.8075) (width 0.25) (layer "F.Cu") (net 1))
 (segment (start 159.125 92.125) (end 160.05 91.2) (width 0.25) (layer "F.Cu") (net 1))
 (segment (start 163.614801 80.765001) (end 162.805901 80.765001) (width 0.25) (layer "F.Cu") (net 1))
 (segment (start 159.6 92.6) (end 159.6 93.1925) (width 0.25) (layer "F.Cu") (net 1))
 (segment (start 138.23202 90.68798) (end 137.87 91.05) (width 0.25) (layer "F.Cu") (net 1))
 (segment (start 164.240006 98.65) (end 163.75 98.65) (width 0.25) (layer "F.Cu") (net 1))
 (segment (start 161.497139 94.0075) (end 161.6 94.0075) (width 0.25) (layer "F.Cu") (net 1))
 (segment (start 158.731 92.519) (end 159.125 92.125) (width 0.25) (layer "F.Cu") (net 1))
 (segment (start 163.614801 84.765001) (end 163.689312 84.69049) (width 0.25) (layer "F.Cu") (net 1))
 (segment (start 137.785 86.1) (end 137.785 87.0725) (width 0.25) (layer "F.Cu") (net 1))
 (segment (start 137.785 87.0725) (end 137.6075 87.25) (width 0.25) (layer "F.Cu") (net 1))
 (segment (start 161.6 94.0075) (end 162.597506 94.0075) (width 0.25) (layer "F.Cu") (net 1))
 (segment (start 137.87 91.05) (end 136.6 91.05) (width 0.25) (layer "F.Cu") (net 1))
 (segment (start 164.49952 95.909514) (end 164.49952 98.390486) (width 0.25) (layer "F.Cu") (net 1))
 (segment (start 156.798978 92.519) (end 157.628 92.519) (width 0.25) (layer "F.Cu") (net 1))
 (segment (start 137.565 85.05) (end 137.565 85.88) (width 0.25) (layer "F.Cu") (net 1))
 (segment (start 163.689312 84.69049) (end 163.689312 80.839512) (width 0.25) (layer "F.Cu") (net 1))
 (segment (start 162.805901 84.765001) (end 163.614801 84.765001) (width 0.25) (layer "F.Cu") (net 1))
 (segment (start 137.615 82.95) (end 138.23202 83.56702) (width 0.25) (layer "F.Cu") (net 1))
 (segment (start 138.23202 83.56702) (end 138.23202 84.38298) (width 0.25) (layer "F.Cu") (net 1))
 (segment (start 156.303489 92.023511) (end 156.798978 92.519) (width 0.25) (layer "F.Cu") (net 1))
 (segment (start 156.303489 91.115467) (end 156.303489 92.023511) (width 0.25) (layer "F.Cu") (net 1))
 (segment (start 160.05 88.8075) (end 159.5 88.2575) (width 0.25) (layer "F.Cu") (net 1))
 (segment (start 160.682139 93.1925) (end 161.497139 94.0075) (width 0.25) (layer "F.Cu") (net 1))
 (segment (start 140.628 82.359) (end 147.547022 82.359) (width 0.25) (layer "F.Cu") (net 1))
 (segment (start 159.5 88.2575) (end 159.755643 88.2575) (width 0.25) (layer "F.Cu") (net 1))
 (segment (start 137.565 85.88) (end 137.785 86.1) (width 0.25) (layer "F.Cu") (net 1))
 (segment (start 163.689312 80.839512) (end 163.614801 80.765001) (width 0.25) (layer "F.Cu") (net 1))
 (segment (start 157.628 92.519) (end 158.731 92.519) (width 0.25) (layer "F.Cu") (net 1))
 (segment (start 137.59 88.25) (end 138.23202 88.89202) (width 0.25) (layer "F.Cu") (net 1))
 (segment (start 159.125 92.125) (end 159.6 92.6) (width 0.25) (layer "F.Cu") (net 1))
 (segment (start 138.23202 88.89202) (end 138.23202 90.68798) (width 0.25) (layer "F.Cu") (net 1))
 (segment (start 159.6 93.1925) (end 160.682139 93.1925) (width 0.25) (layer "F.Cu") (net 1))
 (segment (start 159.755643 88.2575) (end 162.805901 85.207242) (width 0.25) (layer "F.Cu") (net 1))
 (segment (start 138.0625 82.5025) (end 137.615 82.95) (width 0.25) (layer "F.Cu") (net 1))
 (segment (start 137.6075 87.25) (end 137.6075 88.2325) (width 0.25) (layer "F.Cu") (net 1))
 (segment (start 138.23202 84.38298) (end 137.565 85.05) (width 0.25) (layer "F.Cu") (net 1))
 (segment (start 164.49952 98.390486) (end 164.240006 98.65) (width 0.25) (layer "F.Cu") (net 1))
 (segment (start 162.805901 85.207242) (end 162.805901 84.765001) (width 0.25) (layer "F.Cu") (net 1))
 (segment (start 138.0625 81.05) (end 138.0625 82.5025) (width 0.25) (layer "F.Cu") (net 1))
 (segment (start 147.547022 82.359) (end 156.303489 91.115467) (width 0.25) (layer "F.Cu") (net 1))
 (segment (start 137.6075 88.2325) (end 137.59 88.25) (width 0.25) (layer "F.Cu") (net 1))
 (segment (start 162.597506 94.0075) (end 164.49952 95.909514) (width 0.25) (layer "F.Cu") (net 1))
 (segment (start 138.0625 82.5025) (end 138.206 82.359) (width 0.25) (layer "F.Cu") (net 1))
 (segment (start 136.6 95.9) (end 138 94.5) (width 0.25) (layer "F.Cu") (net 6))
 (segment (start 136.6 97.355) (end 136.6 96.4983) (width 0.25) (layer "F.Cu") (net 6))
 (segment (start 135.755 98.2) (end 136.6 97.355) (width 0.25) (layer "F.Cu") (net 6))
 (segment (start 136.6 96.4983) (end 136.6 95.9) (width 0.25) (layer "F.Cu") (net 6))
 (segment (start 136.6 96.4983) (end 137.87 96.4983) (width 0.25) (layer "F.Cu") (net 6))
 (via (at 138 94.5) (size 0.8) (drill 0.4) (layers "F.Cu" "B.Cu") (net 6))
 (segment (start 138 94.5) (end 136.7 93.2) (width 0.25) (layer "B.Cu") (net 6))
 (segment (start 136.7 93.2) (end 135.95 93.2) (width 0.25) (layer "B.Cu") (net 6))
 (segment (start 144 97.15) (end 137.95 97.15) (width 0.25) (layer "B.Cu") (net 7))
 (segment (start 137.95 97.15) (end 136.9 98.2) (width 0.25) (layer "B.Cu") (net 7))
 (segment (start 134.06 96.39) (end 134.06 96.4983) (width 0.25) (layer "B.Cu") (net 16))
 (segment (start 135.95 94.5) (end 134.06 96.39) (width 0.25) (layer "B.Cu") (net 16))
 (segment (start 159.613589 80.314489) (end 156.303489 80.314489) (width 0.25) (layer "F.Cu") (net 10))
 (segment (start 156.16187 80.456108) (end 156.16187 89.66187) (width 0.25) (layer "F.Cu") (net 10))
 (segment (start 156.303489 80.314489) (end 156.16187 80.456108) (width 0.25) (layer "F.Cu") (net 10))
 (segment (start 160.064099 80.764999) (end 159.613589 80.314489) (width 0.25) (layer "F.Cu") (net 10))
 (segment (start 156.16187 89.66187) (end 156.479 89.979) (width 0.25) (layer "F.Cu") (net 10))
 (segment (start 156.479 89.979) (end 157.628 89.979) (width 0.25) (layer "F.Cu") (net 10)))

